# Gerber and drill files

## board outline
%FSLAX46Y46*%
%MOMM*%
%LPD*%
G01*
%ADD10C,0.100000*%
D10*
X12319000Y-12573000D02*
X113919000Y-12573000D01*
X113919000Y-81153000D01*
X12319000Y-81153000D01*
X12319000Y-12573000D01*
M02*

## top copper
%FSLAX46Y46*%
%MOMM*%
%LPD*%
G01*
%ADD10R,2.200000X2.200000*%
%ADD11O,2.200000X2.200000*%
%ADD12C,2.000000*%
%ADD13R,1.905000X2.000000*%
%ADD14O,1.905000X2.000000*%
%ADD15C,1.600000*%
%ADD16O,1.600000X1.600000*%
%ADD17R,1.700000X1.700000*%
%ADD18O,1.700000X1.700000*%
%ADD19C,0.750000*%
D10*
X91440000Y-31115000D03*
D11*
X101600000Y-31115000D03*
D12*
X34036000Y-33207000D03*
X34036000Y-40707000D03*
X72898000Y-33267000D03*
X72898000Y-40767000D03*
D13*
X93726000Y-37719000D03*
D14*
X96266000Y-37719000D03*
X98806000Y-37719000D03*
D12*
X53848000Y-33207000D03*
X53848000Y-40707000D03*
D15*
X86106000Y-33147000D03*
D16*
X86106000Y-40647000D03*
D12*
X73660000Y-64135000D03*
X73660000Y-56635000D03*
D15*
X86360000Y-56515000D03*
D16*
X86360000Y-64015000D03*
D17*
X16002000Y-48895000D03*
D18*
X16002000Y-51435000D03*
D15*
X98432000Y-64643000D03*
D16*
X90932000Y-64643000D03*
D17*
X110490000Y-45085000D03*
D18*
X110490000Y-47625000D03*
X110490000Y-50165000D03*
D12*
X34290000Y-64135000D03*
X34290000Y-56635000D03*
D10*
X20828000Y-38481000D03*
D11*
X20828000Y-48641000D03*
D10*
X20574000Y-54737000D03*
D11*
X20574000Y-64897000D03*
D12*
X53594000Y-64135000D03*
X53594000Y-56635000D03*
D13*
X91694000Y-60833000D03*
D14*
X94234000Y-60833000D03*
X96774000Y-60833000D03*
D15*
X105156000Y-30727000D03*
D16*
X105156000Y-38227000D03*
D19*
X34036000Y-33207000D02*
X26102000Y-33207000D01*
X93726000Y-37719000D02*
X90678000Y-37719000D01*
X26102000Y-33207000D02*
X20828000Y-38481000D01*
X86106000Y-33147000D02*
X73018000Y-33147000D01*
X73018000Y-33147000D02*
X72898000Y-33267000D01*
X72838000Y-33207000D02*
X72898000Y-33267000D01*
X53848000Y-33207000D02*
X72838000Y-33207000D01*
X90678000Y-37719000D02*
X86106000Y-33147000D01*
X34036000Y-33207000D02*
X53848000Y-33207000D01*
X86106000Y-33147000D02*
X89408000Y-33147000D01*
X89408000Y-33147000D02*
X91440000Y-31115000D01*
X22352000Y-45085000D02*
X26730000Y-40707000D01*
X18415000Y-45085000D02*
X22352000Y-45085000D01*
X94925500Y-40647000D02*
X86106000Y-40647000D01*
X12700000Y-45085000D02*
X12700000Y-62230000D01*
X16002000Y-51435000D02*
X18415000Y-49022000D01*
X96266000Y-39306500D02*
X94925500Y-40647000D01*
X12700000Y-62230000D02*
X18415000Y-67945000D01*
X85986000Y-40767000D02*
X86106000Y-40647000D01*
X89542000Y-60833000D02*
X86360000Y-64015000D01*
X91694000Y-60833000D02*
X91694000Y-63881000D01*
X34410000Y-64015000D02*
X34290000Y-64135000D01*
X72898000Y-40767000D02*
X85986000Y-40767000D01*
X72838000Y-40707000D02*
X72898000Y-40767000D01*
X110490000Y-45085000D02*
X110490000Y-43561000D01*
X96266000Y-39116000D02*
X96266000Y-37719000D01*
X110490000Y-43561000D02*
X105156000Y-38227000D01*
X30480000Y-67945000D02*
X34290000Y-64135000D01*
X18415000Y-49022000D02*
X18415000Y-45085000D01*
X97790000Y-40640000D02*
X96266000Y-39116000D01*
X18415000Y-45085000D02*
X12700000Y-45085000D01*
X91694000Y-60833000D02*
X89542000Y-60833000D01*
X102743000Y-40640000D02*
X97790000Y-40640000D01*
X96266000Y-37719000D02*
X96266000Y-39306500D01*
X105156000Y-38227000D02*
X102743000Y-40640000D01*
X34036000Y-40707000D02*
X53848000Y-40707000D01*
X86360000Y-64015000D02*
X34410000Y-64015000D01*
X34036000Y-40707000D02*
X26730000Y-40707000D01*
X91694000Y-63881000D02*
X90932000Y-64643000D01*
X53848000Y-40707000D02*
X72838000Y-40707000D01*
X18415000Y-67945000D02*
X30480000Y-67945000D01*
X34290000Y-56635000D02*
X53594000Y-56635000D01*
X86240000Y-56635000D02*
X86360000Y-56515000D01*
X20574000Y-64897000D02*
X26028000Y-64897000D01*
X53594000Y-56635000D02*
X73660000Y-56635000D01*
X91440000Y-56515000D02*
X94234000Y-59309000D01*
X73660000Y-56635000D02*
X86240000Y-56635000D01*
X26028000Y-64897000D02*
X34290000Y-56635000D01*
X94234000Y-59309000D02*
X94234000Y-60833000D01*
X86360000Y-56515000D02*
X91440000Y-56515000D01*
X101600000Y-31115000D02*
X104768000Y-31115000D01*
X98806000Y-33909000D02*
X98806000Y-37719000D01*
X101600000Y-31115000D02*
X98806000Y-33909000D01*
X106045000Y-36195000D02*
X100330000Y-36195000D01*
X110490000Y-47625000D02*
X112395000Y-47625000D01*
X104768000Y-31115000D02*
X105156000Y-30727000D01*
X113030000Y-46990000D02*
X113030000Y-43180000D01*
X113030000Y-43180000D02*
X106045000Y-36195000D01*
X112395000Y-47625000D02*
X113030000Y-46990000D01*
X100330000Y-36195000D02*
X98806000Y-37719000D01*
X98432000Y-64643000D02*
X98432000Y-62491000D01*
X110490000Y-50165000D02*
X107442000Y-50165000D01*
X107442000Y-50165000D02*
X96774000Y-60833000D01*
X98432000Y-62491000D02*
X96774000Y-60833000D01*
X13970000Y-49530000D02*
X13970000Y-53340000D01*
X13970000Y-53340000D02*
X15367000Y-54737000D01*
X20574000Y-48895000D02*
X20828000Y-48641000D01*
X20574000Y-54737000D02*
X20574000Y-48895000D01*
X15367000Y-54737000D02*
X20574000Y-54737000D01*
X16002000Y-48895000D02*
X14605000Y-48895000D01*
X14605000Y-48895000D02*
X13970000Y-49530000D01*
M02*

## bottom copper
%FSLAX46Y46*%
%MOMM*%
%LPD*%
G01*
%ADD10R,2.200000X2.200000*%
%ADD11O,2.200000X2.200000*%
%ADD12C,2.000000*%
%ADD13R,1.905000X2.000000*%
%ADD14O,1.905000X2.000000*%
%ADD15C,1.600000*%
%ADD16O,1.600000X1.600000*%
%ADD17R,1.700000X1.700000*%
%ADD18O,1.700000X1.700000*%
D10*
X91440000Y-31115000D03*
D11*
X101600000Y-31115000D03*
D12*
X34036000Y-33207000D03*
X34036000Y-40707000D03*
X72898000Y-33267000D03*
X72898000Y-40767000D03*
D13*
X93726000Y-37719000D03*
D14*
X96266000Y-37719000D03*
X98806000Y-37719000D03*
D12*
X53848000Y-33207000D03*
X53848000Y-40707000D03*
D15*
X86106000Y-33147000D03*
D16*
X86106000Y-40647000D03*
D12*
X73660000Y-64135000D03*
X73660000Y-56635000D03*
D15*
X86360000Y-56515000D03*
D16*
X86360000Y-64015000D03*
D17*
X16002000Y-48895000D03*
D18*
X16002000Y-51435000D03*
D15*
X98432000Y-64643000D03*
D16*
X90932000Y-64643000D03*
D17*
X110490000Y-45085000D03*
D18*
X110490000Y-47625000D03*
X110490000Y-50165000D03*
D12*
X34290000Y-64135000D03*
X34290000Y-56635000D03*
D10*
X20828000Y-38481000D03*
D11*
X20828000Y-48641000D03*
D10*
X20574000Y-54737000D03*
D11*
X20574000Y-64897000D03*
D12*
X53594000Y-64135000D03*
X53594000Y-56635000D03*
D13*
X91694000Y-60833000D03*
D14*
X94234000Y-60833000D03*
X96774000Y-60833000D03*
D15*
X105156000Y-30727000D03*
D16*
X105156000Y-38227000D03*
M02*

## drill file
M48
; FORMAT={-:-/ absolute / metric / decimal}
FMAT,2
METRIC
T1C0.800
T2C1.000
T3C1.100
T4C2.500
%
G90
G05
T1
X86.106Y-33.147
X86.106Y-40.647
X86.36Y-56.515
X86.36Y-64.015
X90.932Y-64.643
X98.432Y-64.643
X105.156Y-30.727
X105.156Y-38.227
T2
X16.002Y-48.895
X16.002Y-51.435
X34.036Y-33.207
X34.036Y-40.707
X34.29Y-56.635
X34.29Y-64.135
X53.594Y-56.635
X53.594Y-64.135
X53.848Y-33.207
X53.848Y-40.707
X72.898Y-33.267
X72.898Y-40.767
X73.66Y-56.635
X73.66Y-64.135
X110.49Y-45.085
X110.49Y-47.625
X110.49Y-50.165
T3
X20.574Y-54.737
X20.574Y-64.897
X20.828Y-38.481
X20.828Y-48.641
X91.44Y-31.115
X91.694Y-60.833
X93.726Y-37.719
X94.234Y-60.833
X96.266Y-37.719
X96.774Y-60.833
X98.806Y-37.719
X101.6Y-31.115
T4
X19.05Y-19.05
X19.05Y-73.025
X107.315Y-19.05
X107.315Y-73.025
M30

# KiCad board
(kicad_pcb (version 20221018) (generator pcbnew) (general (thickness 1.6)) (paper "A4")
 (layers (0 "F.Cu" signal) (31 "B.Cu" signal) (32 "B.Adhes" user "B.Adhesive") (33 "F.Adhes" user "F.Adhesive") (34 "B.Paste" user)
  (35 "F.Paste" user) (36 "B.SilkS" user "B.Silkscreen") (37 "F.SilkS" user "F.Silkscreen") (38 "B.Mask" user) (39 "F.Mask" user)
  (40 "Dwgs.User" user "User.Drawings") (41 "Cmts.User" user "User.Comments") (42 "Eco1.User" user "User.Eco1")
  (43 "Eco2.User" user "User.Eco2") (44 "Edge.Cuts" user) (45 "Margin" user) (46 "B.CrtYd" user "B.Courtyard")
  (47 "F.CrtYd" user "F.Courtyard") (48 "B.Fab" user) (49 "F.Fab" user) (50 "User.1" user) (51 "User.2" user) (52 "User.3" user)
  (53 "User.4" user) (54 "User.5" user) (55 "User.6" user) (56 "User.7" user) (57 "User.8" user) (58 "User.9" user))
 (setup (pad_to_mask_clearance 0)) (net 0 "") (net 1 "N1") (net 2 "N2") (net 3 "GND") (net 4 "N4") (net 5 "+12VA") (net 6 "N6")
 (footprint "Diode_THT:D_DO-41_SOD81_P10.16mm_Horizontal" (layer "F.Cu") (at 91.44 31.115)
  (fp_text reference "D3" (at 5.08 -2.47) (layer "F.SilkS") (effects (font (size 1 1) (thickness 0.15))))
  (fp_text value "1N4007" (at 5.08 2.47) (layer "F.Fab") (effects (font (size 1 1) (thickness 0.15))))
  (pad "1" thru_hole rect (at 0 0) (size 2.2 2.2) (drill 1.1) (layers "*.Cu" "*.Mask") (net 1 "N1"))
  (pad "2" thru_hole oval (at 10.16 0) (size 2.2 2.2) (drill 1.1) (layers "*.Cu" "*.Mask") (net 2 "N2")))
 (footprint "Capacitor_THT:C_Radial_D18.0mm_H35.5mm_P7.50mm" (layer "F.Cu") (at 34.036 33.207 -90)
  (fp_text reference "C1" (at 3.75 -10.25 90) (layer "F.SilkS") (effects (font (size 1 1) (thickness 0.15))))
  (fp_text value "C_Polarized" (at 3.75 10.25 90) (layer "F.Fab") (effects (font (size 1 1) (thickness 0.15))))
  (pad "1" thru_hole circle (at 0 0 270) (size 2 2) (drill 1) (layers "*.Cu" "*.Mask") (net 1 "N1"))
  (pad "2" thru_hole circle (at 7.5 0 270) (size 2 2) (drill 1) (layers "*.Cu" "*.Mask") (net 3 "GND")))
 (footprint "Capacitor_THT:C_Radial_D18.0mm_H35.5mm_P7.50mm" (layer "F.Cu") (at 72.898 33.267 -90)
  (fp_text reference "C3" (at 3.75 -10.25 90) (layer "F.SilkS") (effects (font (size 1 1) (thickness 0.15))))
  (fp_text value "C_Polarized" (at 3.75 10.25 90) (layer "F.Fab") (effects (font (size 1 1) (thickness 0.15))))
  (pad "1" thru_hole circle (at 0 0 270) (size 2 2) (drill 1) (layers "*.Cu" "*.Mask") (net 1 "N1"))
  (pad "2" thru_hole circle (at 7.5 0 270) (size 2 2) (drill 1) (layers "*.Cu" "*.Mask") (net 3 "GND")))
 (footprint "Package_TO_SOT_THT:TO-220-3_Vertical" (layer "F.Cu") (at 93.726 37.719)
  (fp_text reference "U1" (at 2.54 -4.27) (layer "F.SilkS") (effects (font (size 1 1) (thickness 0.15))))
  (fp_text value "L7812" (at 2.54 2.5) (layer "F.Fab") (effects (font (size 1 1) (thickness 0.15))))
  (pad "1" thru_hole rect (at 0 0) (size 1.905 2) (drill 1.1) (layers "*.Cu" "*.Mask") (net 1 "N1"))
  (pad "2" thru_hole oval (at 2.54 0) (size 1.905 2) (drill 1.1) (layers "*.Cu" "*.Mask") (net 3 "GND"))
  (pad "3" thru_hole oval (at 5.08 0) (size 1.905 2) (drill 1.1) (layers "*.Cu" "*.Mask") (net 2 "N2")))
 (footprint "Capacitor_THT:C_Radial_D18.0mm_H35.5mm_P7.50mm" (layer "F.Cu") (at 53.848 33.207 -90)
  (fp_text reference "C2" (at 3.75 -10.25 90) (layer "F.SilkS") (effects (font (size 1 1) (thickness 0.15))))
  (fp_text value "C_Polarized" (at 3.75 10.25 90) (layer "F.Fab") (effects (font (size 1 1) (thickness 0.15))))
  (pad "1" thru_hole circle (at 0 0 270) (size 2 2) (drill 1) (layers "*.Cu" "*.Mask") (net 1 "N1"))
  (pad "2" thru_hole circle (at 7.5 0 270) (size 2 2) (drill 1) (layers "*.Cu" "*.Mask") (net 3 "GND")))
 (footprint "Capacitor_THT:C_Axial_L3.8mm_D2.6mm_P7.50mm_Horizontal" (layer "F.Cu") (at 86.106 33.147 -90)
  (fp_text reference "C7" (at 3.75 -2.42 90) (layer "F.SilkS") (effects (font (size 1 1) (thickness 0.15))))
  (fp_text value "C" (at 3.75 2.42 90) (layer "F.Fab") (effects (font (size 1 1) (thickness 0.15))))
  (pad "1" thru_hole circle (at 0 0 270) (size 1.6 1.6) (drill 0.8) (layers "*.Cu" "*.Mask") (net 1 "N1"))
  (pad "2" thru_hole oval (at 7.5 0 270) (size 1.6 1.6) (drill 0.8) (layers "*.Cu" "*.Mask") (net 3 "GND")))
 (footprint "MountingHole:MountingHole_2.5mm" (layer "F.Cu") (at 19.05 19.05)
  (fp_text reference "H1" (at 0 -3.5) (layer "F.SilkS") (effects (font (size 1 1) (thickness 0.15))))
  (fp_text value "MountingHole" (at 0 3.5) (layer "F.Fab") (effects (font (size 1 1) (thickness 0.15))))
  (pad "" np_thru_hole circle (at 0 0) (size 2.5 2.5) (drill 2.5) (layers "*.Cu" "*.Mask")))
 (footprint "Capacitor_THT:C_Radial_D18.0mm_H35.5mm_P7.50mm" (layer "F.Cu") (at 73.66 64.135 90)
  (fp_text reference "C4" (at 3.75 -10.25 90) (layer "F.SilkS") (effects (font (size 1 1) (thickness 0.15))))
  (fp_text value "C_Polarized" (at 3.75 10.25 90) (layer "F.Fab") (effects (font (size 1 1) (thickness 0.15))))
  (pad "1" thru_hole circle (at 0 0 90) (size 2 2) (drill 1) (layers "*.Cu" "*.Mask") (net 3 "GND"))
  (pad "2" thru_hole circle (at 7.5 0 90) (size 2 2) (drill 1) (layers "*.Cu" "*.Mask") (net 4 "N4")))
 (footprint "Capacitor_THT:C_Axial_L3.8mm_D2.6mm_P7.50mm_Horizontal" (layer "F.Cu") (at 86.36 56.515 -90)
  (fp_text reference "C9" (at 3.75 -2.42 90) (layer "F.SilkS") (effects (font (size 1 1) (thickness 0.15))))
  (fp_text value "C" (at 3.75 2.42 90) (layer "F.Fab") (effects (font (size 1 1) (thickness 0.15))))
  (pad "1" thru_hole circle (at 0 0 270) (size 1.6 1.6) (drill 0.8) (layers "*.Cu" "*.Mask") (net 4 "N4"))
  (pad "2" thru_hole oval (at 7.5 0 270) (size 1.6 1.6) (drill 0.8) (layers "*.Cu" "*.Mask") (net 3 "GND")))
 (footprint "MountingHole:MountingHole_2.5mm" (layer "F.Cu") (at 19.05 73.025)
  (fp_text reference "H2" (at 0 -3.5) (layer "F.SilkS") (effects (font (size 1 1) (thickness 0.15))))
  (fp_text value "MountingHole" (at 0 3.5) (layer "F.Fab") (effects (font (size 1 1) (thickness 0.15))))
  (pad "" np_thru_hole circle (at 0 0) (size 2.5 2.5) (drill 2.5) (layers "*.Cu" "*.Mask")))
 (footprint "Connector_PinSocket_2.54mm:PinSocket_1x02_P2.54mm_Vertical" (layer "F.Cu") (at 16.002 48.895)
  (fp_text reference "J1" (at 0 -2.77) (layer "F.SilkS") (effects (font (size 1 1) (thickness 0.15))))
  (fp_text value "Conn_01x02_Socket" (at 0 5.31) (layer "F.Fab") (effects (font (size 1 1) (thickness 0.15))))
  (pad "1" thru_hole rect (at 0 0) (size 1.7 1.7) (drill 1) (layers "*.Cu" "*.Mask") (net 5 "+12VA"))
  (pad "2" thru_hole oval (at 0 2.54) (size 1.7 1.7) (drill 1) (layers "*.Cu" "*.Mask") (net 3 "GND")))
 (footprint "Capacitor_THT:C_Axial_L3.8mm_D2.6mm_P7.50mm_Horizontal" (layer "F.Cu") (at 98.432 64.643 180)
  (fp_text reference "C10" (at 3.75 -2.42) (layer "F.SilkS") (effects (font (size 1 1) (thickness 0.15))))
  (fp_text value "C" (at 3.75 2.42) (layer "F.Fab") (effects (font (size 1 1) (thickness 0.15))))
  (pad "1" thru_hole circle (at 0 0 180) (size 1.6 1.6) (drill 0.8) (layers "*.Cu" "*.Mask") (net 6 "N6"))
  (pad "2" thru_hole oval (at 7.5 0 180) (size 1.6 1.6) (drill 0.8) (layers "*.Cu" "*.Mask") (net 3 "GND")))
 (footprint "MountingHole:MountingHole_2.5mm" (layer "F.Cu") (at 107.315 73.025)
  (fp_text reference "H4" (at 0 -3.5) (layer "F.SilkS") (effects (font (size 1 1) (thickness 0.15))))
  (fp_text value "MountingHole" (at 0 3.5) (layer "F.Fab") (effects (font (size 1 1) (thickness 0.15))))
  (pad "" np_thru_hole circle (at 0 0) (size 2.5 2.5) (drill 2.5) (layers "*.Cu" "*.Mask")))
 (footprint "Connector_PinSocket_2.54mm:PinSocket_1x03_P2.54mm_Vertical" (layer "F.Cu") (at 110.49 45.085)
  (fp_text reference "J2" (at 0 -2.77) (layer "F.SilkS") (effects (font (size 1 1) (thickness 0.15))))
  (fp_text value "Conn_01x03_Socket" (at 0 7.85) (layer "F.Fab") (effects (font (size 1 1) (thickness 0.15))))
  (pad "1" thru_hole rect (at 0 0) (size 1.7 1.7) (drill 1) (layers "*.Cu" "*.Mask") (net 3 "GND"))
  (pad "2" thru_hole oval (at 0 2.54) (size 1.7 1.7) (drill 1) (layers "*.Cu" "*.Mask") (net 2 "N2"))
  (pad "3" thru_hole oval (at 0 5.08) (size 1.7 1.7) (drill 1) (layers "*.Cu" "*.Mask") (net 6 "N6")))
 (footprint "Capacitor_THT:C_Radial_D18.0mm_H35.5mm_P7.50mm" (layer "F.Cu") (at 34.29 64.135 90)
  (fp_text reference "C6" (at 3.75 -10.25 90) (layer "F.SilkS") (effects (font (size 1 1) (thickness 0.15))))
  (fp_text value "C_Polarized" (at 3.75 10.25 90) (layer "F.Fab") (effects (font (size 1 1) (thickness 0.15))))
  (pad "1" thru_hole circle (at 0 0 90) (size 2 2) (drill 1) (layers "*.Cu" "*.Mask") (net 3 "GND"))
  (pad "2" thru_hole circle (at 7.5 0 90) (size 2 2) (drill 1) (layers "*.Cu" "*.Mask") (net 4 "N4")))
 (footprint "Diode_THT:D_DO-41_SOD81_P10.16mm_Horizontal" (layer "F.Cu") (at 20.828 38.481 -90)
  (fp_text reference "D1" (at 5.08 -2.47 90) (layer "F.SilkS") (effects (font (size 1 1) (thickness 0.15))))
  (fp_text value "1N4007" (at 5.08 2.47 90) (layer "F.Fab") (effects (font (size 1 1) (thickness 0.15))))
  (pad "1" thru_hole rect (at 0 0 270) (size 2.2 2.2) (drill 1.1) (layers "*.Cu" "*.Mask") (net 1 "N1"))
  (pad "2" thru_hole oval (at 10.16 0 270) (size 2.2 2.2) (drill 1.1) (layers "*.Cu" "*.Mask") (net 5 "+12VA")))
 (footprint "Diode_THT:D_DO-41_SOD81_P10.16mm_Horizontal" (layer "F.Cu") (at 20.574 54.737 -90)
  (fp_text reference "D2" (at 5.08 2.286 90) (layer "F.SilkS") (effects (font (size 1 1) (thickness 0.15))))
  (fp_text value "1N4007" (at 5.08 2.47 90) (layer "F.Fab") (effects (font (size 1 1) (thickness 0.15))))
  (pad "1" thru_hole rect (at 0 0 270) (size 2.2 2.2) (drill 1.1) (layers "*.Cu" "*.Mask") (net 5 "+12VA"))
  (pad "2" thru_hole oval (at 10.16 0 270) (size 2.2 2.2) (drill 1.1) (layers "*.Cu" "*.Mask") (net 4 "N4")))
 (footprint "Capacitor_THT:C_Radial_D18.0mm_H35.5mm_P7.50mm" (layer "F.Cu") (at 53.594 64.135 90)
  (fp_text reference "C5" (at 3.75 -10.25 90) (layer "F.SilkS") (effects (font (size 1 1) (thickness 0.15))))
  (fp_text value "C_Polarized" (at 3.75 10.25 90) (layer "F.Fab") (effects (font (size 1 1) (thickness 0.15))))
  (pad "1" thru_hole circle (at 0 0 90) (size 2 2) (drill 1) (layers "*.Cu" "*.Mask") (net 3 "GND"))
  (pad "2" thru_hole circle (at 7.5 0 90) (size 2 2) (drill 1) (layers "*.Cu" "*.Mask") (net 4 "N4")))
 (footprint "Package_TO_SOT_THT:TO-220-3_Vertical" (layer "F.Cu") (at 91.694 60.833)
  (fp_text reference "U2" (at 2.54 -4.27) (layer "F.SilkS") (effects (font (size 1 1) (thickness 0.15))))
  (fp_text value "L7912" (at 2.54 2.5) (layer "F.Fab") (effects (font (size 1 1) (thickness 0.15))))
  (pad "1" thru_hole rect (at 0 0) (size 1.905 2) (drill 1.1) (layers "*.Cu" "*.Mask") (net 3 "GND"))
  (pad "2" thru_hole oval (at 2.54 0) (size 1.905 2) (drill 1.1) (layers "*.Cu" "*.Mask") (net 4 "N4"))
  (pad "3" thru_hole oval (at 5.08 0) (size 1.905 2) (drill 1.1) (layers "*.Cu" "*.Mask") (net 6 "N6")))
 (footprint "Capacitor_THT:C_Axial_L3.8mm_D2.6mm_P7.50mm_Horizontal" (layer "F.Cu") (at 105.156 30.727 -90)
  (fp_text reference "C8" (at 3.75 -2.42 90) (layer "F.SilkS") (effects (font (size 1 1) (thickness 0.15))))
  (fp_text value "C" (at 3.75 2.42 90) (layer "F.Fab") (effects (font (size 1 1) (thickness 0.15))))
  (pad "1" thru_hole circle (at 0 0 270) (size 1.6 1.6) (drill 0.8) (layers "*.Cu" "*.Mask") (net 2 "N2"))
  (pad "2" thru_hole oval (at 7.5 0 270) (size 1.6 1.6) (drill 0.8) (layers "*.Cu" "*.Mask") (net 3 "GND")))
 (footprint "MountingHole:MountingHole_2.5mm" (layer "F.Cu") (at 107.315 19.05)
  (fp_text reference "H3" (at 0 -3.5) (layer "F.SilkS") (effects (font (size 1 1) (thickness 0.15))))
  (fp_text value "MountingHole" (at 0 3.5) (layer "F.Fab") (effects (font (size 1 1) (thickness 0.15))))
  (pad "" np_thru_hole circle (at 0 0) (size 2.5 2.5) (drill 2.5) (layers "*.Cu" "*.Mask")))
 (gr_rect (start 12.319 12.573) (end 113.919 81.153) (stroke (width 0.1) (type default)) (fill none) (layer "Edge.Cuts"))
 (segment (start 34.036 33.207) (end 26.102 33.207) (width 0.75) (layer "F.Cu") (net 1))
 (segment (start 93.726 37.719) (end 90.678 37.719) (width 0.75) (layer "F.Cu") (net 1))
 (segment (start 26.102 33.207) (end 20.828 38.481) (width 0.75) (layer "F.Cu") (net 1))
 (segment (start 86.106 33.147) (end 73.018 33.147) (width 0.75) (layer "F.Cu") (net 1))
 (segment (start 73.018 33.147) (end 72.898 33.267) (width 0.75) (layer "F.Cu") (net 1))
 (segment (start 72.838 33.207) (end 72.898 33.267) (width 0.75) (layer "F.Cu") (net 1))
 (segment (start 53.848 33.207) (end 72.838 33.207) (width 0.75) (layer "F.Cu") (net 1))
 (segment (start 90.678 37.719) (end 86.106 33.147) (width 0.75) (layer "F.Cu") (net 1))
 (segment (start 34.036 33.207) (end 53.848 33.207) (width 0.75) (layer "F.Cu") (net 1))
 (segment (start 86.106 33.147) (end 89.408 33.147) (width 0.75) (layer "F.Cu") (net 1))
 (segment (start 89.408 33.147) (end 91.44 31.115) (width 0.75) (layer "F.Cu") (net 1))
 (segment (start 22.352 45.085) (end 26.73 40.707) (width 0.75) (layer "F.Cu") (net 3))
 (segment (start 18.415 45.085) (end 22.352 45.085) (width 0.75) (layer "F.Cu") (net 3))
 (segment (start 94.9255 40.647) (end 86.106 40.647) (width 0.75) (layer "F.Cu") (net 3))
 (segment (start 12.7 45.085) (end 12.7 62.23) (width 0.75) (layer "F.Cu") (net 3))
 (segment (start 16.002 51.435) (end 18.415 49.022) (width 0.75) (layer "F.Cu") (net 3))
 (segment (start 96.266 39.3065) (end 94.9255 40.647) (width 0.75) (layer "F.Cu") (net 3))
 (segment (start 12.7 62.23) (end 18.415 67.945) (width 0.75) (layer "F.Cu") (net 3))
 (segment (start 85.986 40.767) (end 86.106 40.647) (width 0.75) (layer "F.Cu") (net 3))
 (segment (start 89.542 60.833) (end 86.36 64.015) (width 0.75) (layer "F.Cu") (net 3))
 (segment (start 91.694 60.833) (end 91.694 63.881) (width 0.75) (layer "F.Cu") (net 3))
 (segment (start 34.41 64.015) (end 34.29 64.135) (width 0.75) (layer "F.Cu") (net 3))
 (segment (start 72.898 40.767) (end 85.986 40.767) (width 0.75) (layer "F.Cu") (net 3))
 (segment (start 72.838 40.707) (end 72.898 40.767) (width 0.75) (layer "F.Cu") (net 3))
 (segment (start 110.49 45.085) (end 110.49 43.561) (width 0.75) (layer "F.Cu") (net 3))
 (segment (start 96.266 39.116) (end 96.266 37.719) (width 0.75) (layer "F.Cu") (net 3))
 (segment (start 110.49 43.561) (end 105.156 38.227) (width 0.75) (layer "F.Cu") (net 3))
 (segment (start 30.48 67.945) (end 34.29 64.135) (width 0.75) (layer "F.Cu") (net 3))
 (segment (start 18.415 49.022) (end 18.415 45.085) (width 0.75) (layer "F.Cu") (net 3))
 (segment (start 97.79 40.64) (end 96.266 39.116) (width 0.75) (layer "F.Cu") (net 3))
 (segment (start 18.415 45.085) (end 12.7 45.085) (width 0.75) (layer "F.Cu") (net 3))
 (segment (start 91.694 60.833) (end 89.542 60.833) (width 0.75) (layer "F.Cu") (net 3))
 (segment (start 102.743 40.64) (end 97.79 40.64) (width 0.75) (layer "F.Cu") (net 3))
 (segment (start 96.266 37.719) (end 96.266 39.3065) (width 0.75) (layer "F.Cu") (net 3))
 (segment (start 105.156 38.227) (end 102.743 40.64) (width 0.75) (layer "F.Cu") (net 3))
 (segment (start 34.036 40.707) (end 53.848 40.707) (width 0.75) (layer "F.Cu") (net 3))
 (segment (start 86.36 64.015) (end 34.41 64.015) (width 0.75) (layer "F.Cu") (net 3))
 (segment (start 34.036 40.707) (end 26.73 40.707) (width 0.75) (layer "F.Cu") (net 3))
 (segment (start 91.694 63.881) (end 90.932 64.643) (width 0.75) (layer "F.Cu") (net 3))
 (segment (start 53.848 40.707) (end 72.838 40.707) (width 0.75) (layer "F.Cu") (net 3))
 (segment (start 18.415 67.945) (end 30.48 67.945) (width 0.75) (layer "F.Cu") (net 3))
 (segment (start 34.29 56.635) (end 53.594 56.635) (width 0.75) (layer "F.Cu") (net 4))
 (segment (start 86.24 56.635) (end 86.36 56.515) (width 0.75) (layer "F.Cu") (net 4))
 (segment (start 20.574 64.897) (end 26.028 64.897) (width 0.75) (layer "F.Cu") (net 4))
 (segment (start 53.594 56.635) (end 73.66 56.635) (width 0.75) (layer "F.Cu") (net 4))
 (segment (start 91.44 56.515) (end 94.234 59.309) (width 0.75) (layer "F.Cu") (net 4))
 (segment (start 73.66 56.635) (end 86.24 56.635) (width 0.75) (layer "F.Cu") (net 4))
 (segment (start 26.028 64.897) (end 34.29 56.635) (width 0.75) (layer "F.Cu") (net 4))
 (segment (start 94.234 59.309) (end 94.234 60.833) (width 0.75) (layer "F.Cu") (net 4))
 (segment (start 86.36 56.515) (end 91.44 56.515) (width 0.75) (layer "F.Cu") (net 4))
 (segment (start 101.6 31.115) (end 104.768 31.115) (width 0.75) (layer "F.Cu") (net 2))
 (segment (start 98.806 33.909) (end 98.806 37.719) (width 0.75) (layer "F.Cu") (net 2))
 (segment (start 101.6 31.115) (end 98.806 33.909) (width 0.75) (layer "F.Cu") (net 2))
 (segment (start 106.045 36.195) (end 100.33 36.195) (width 0.75) (layer "F.Cu") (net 2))
 (segment (start 110.49 47.625) (end 112.395 47.625) (width 0.75) (layer "F.Cu") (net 2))
 (segment (start 104.768 31.115) (end 105.156 30.727) (width 0.75) (layer "F.Cu") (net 2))
 (segment (start 113.03 46.99) (end 113.03 43.18) (width 0.75) (layer "F.Cu") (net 2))
 (segment (start 113.03 43.18) (end 106.045 36.195) (width 0.75) (layer "F.Cu") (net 2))
 (segment (start 112.395 47.625) (end 113.03 46.99) (width 0.75) (layer "F.Cu") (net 2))
 (segment (start 100.33 36.195) (end 98.806 37.719) (width 0.75) (layer "F.Cu") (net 2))
 (segment (start 98.432 64.643) (end 98.432 62.491) (width 0.75) (layer "F.Cu") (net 6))
 (segment (start 110.49 50.165) (end 107.442 50.165) (width 0.75) (layer "F.Cu") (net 6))
 (segment (start 107.442 50.165) (end 96.774 60.833) (width 0.75) (layer "F.Cu") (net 6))
 (segment (start 98.432 62.491) (end 96.774 60.833) (width 0.75) (layer "F.Cu") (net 6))
 (segment (start 13.97 49.53) (end 13.97 53.34) (width 0.75) (layer "F.Cu") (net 5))
 (segment (start 13.97 53.34) (end 15.367 54.737) (width 0.75) (layer "F.Cu") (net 5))
 (segment (start 20.574 48.895) (end 20.828 48.641) (width 0.75) (layer "F.Cu") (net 5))
 (segment (start 20.574 54.737) (end 20.574 48.895) (width 0.75) (layer "F.Cu") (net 5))
 (segment (start 15.367 54.737) (end 20.574 54.737) (width 0.75) (layer "F.Cu") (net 5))
 (segment (start 16.002 48.895) (end 14.605 48.895) (width 0.75) (layer "F.Cu") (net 5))
 (segment (start 14.605 48.895) (end 13.97 49.53) (width 0.75) (layer "F.Cu") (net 5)))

